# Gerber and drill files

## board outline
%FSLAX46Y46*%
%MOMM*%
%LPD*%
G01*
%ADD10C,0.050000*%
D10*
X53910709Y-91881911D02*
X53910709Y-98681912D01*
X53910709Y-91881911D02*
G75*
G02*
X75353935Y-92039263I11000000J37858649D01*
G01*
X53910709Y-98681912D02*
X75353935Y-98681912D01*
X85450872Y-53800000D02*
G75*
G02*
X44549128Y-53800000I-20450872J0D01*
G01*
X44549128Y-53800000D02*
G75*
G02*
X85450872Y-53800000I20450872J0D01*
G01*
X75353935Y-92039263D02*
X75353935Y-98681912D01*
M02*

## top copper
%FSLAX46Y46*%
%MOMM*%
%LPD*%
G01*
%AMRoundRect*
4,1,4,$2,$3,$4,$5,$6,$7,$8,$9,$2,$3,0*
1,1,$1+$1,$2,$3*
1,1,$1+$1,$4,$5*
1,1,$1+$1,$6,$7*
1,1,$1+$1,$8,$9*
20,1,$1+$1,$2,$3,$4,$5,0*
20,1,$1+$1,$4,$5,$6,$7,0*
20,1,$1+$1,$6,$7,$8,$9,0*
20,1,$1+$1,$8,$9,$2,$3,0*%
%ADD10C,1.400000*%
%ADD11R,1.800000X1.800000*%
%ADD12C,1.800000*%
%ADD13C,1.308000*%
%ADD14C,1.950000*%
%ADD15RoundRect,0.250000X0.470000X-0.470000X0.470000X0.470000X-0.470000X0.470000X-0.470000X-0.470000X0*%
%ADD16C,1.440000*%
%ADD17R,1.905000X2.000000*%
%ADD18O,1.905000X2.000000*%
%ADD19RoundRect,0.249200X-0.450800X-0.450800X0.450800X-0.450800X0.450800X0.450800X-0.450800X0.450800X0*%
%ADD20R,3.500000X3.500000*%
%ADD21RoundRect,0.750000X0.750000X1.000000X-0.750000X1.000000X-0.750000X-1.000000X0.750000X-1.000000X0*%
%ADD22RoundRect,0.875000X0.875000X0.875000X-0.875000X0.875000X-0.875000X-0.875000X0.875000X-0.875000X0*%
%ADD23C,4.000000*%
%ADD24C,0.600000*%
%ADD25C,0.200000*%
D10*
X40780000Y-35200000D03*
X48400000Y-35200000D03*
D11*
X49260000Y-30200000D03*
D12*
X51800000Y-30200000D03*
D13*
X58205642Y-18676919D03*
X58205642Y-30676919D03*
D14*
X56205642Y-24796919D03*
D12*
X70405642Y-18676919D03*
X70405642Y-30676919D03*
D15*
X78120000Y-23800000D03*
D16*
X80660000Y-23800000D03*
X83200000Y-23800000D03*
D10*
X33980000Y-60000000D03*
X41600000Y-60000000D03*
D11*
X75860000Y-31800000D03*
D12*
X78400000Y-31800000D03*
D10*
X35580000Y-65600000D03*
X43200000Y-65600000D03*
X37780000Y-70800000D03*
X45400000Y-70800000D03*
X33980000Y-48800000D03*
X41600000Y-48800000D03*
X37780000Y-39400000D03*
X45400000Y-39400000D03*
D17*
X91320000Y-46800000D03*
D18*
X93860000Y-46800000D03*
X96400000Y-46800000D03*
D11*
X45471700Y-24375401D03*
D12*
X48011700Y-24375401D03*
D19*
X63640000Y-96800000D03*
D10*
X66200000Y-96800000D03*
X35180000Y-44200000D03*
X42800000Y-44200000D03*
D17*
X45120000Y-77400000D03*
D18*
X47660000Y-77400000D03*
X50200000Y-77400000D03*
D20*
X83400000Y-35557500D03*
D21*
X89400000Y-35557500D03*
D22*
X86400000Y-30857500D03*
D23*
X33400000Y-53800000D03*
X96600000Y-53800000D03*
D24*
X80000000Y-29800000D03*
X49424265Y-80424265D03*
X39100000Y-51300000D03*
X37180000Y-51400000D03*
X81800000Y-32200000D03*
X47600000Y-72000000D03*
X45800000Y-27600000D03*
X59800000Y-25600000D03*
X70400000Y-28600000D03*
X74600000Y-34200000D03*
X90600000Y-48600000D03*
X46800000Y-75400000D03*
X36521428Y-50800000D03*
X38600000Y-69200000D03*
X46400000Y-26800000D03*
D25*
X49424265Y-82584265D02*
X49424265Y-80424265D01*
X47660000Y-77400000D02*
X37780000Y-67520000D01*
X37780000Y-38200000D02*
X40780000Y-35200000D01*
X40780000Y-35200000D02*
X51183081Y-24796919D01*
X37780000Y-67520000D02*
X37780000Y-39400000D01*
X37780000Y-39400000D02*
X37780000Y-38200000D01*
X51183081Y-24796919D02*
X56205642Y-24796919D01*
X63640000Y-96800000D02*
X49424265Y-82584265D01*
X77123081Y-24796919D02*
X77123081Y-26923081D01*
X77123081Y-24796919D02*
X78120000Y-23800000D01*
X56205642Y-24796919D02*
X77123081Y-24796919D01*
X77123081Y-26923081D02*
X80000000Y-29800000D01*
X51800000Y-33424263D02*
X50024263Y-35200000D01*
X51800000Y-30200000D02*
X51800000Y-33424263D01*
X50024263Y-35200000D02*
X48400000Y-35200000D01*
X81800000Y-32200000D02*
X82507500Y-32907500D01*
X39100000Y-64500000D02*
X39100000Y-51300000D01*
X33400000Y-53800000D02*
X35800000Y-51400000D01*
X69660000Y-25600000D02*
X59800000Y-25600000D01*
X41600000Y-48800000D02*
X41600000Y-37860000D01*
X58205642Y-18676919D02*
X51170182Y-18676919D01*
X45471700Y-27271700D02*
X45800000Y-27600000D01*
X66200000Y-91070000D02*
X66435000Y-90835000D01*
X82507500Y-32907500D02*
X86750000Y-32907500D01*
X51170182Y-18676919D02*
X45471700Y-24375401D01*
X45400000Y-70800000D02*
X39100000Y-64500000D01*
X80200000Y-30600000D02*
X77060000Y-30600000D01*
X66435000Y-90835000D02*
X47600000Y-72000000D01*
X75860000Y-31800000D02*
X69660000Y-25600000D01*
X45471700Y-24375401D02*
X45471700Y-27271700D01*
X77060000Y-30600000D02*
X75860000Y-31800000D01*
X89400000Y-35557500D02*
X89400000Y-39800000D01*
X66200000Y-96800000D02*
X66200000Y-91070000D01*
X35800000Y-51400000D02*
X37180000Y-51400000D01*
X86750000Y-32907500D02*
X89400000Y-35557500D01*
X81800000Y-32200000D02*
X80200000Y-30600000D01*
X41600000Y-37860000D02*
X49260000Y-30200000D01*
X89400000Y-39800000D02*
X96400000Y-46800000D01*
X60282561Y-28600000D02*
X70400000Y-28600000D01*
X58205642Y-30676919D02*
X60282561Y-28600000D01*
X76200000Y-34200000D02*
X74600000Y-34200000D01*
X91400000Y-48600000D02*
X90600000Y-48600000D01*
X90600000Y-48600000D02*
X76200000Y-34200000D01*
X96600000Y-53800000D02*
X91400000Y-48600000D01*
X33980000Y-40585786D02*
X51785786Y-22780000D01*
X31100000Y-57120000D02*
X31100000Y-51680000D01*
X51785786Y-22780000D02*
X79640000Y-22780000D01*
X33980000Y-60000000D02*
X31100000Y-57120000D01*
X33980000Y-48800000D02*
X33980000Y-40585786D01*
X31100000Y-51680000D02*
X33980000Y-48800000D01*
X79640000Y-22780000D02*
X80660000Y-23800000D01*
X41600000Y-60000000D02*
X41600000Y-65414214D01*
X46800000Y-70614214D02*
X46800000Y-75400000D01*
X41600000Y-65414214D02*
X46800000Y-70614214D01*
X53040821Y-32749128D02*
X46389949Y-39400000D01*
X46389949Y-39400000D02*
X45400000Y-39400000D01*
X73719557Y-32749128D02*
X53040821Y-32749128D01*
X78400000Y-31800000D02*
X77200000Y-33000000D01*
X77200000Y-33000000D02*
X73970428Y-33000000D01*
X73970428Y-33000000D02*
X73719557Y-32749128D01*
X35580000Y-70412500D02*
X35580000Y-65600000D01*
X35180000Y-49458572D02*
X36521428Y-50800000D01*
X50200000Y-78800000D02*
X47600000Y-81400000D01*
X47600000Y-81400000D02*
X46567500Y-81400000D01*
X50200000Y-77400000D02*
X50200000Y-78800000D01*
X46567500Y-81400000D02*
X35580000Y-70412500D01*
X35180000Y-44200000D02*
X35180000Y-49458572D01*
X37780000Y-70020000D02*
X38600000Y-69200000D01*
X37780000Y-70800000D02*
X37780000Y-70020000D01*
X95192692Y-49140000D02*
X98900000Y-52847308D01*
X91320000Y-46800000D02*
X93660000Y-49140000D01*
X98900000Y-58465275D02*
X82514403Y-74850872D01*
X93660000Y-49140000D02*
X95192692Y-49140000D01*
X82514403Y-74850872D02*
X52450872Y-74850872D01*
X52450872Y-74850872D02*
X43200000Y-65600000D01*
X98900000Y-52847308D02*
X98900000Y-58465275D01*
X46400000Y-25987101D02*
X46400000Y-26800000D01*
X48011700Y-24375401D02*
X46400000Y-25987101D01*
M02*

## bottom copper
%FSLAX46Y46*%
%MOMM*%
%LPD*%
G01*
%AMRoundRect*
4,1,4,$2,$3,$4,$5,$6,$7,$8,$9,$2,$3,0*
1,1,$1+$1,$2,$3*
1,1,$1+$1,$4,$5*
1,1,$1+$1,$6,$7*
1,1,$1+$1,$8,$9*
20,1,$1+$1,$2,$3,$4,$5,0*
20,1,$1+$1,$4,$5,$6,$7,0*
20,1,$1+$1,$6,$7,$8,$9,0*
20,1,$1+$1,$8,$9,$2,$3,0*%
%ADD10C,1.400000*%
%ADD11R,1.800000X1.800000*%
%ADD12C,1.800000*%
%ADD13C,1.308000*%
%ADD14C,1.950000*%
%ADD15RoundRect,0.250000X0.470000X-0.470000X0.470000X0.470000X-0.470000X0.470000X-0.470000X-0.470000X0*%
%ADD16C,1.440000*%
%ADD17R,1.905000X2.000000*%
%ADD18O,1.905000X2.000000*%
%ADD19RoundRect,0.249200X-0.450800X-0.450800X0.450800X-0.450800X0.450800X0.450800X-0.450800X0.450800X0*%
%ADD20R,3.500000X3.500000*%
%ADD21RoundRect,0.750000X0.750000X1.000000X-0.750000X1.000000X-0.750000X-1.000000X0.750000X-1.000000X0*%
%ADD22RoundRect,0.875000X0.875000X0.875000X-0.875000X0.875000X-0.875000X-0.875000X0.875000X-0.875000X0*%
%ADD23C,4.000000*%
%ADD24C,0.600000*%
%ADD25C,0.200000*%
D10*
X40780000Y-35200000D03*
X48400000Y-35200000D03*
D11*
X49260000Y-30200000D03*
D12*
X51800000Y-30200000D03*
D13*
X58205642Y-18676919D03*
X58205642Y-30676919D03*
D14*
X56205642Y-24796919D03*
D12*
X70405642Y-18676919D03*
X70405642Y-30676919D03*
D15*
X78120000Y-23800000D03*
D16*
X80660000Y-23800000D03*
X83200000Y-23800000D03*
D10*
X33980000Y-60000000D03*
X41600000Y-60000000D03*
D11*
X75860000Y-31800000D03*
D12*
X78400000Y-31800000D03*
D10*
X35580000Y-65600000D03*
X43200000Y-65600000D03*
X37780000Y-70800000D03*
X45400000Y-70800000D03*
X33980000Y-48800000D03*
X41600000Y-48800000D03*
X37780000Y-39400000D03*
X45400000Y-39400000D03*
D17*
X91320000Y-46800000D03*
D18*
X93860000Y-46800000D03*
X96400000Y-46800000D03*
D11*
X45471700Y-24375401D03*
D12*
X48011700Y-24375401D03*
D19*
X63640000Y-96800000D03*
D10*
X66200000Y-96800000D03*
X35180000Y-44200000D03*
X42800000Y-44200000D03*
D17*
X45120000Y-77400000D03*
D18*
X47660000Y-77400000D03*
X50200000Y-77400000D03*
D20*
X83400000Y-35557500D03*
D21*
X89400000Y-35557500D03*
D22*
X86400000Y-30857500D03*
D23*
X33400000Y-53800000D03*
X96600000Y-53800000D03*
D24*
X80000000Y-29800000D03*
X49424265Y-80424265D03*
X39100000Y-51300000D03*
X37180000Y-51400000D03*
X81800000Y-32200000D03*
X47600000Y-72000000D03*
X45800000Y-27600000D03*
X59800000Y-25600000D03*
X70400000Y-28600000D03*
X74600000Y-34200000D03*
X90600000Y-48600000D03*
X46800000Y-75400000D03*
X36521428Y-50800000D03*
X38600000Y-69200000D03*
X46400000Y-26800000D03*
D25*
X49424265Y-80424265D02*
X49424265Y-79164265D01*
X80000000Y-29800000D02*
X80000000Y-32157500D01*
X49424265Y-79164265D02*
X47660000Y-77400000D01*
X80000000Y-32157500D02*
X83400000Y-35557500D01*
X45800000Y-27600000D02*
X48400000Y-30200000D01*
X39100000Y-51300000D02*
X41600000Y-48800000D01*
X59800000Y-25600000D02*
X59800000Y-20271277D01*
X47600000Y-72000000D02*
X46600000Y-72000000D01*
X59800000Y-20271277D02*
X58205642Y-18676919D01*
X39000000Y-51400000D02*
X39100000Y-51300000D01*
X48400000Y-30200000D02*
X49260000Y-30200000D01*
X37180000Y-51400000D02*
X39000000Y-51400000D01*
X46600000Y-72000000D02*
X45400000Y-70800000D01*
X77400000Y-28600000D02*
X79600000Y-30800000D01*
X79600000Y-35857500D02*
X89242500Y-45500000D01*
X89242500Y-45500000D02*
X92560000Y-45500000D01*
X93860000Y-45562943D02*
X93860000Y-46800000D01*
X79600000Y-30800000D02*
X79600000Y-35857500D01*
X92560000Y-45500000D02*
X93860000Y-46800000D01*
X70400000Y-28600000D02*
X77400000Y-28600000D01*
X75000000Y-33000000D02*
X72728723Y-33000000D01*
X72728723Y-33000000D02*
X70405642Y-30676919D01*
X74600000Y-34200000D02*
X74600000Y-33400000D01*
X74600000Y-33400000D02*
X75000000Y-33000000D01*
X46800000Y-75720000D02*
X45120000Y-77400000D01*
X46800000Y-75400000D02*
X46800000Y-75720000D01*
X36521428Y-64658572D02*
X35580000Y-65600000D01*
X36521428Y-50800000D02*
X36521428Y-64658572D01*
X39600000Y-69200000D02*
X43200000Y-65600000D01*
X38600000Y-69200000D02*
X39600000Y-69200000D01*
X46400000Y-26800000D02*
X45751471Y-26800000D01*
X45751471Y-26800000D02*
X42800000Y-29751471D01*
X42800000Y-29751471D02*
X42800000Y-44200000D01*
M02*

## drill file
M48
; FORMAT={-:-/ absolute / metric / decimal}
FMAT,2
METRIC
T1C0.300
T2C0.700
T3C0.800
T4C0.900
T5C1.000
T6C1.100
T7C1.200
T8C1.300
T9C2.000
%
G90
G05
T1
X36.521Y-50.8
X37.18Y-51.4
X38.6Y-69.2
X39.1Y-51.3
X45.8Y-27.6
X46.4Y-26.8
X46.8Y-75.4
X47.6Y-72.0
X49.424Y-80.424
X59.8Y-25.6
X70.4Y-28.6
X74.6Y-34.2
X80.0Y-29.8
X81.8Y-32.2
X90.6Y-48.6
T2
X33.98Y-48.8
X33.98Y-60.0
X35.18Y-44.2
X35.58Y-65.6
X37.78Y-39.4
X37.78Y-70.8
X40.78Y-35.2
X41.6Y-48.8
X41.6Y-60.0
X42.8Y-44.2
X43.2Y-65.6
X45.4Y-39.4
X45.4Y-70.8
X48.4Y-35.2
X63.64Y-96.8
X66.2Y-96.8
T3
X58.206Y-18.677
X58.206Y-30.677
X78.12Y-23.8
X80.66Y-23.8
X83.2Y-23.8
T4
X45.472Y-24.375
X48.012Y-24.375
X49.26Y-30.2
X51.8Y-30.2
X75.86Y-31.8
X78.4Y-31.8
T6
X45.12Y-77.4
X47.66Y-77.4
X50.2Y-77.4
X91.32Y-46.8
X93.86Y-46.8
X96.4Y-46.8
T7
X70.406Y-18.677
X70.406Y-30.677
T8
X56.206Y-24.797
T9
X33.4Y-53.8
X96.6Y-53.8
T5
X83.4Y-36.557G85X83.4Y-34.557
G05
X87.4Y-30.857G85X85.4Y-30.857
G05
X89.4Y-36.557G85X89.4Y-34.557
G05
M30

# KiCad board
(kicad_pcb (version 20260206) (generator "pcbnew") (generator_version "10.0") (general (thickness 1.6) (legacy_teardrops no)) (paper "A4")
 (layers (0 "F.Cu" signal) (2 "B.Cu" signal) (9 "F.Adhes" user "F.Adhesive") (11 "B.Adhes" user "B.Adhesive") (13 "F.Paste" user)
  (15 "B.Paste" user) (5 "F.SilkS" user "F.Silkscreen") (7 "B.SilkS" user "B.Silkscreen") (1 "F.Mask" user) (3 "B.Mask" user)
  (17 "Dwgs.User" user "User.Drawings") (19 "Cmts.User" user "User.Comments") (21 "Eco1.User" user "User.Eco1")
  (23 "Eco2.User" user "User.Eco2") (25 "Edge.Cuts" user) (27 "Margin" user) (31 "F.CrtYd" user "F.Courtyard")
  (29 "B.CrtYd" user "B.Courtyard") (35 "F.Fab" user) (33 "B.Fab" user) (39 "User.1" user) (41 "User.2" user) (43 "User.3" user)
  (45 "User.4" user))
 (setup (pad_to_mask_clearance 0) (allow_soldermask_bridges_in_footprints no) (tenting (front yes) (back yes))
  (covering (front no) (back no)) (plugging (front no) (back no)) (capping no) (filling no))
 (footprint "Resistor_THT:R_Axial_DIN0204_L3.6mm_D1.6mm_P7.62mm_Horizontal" (layer "F.Cu") (at 40.78 35.2)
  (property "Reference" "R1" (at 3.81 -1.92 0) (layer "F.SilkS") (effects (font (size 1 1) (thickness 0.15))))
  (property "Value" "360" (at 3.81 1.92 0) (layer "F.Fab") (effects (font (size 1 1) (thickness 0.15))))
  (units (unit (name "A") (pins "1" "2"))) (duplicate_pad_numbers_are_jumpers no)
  (pad "1" thru_hole circle (at 0 0) (size 1.4 1.4) (drill 0.7) (layers "*.Cu" "*.Mask") (remove_unused_layers no) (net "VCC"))
  (pad "2" thru_hole circle (at 7.62 0) (size 1.4 1.4) (drill 0.7) (layers "*.Cu" "*.Mask") (remove_unused_layers no) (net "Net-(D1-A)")))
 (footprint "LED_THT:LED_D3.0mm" (layer "F.Cu") (at 49.26 30.2)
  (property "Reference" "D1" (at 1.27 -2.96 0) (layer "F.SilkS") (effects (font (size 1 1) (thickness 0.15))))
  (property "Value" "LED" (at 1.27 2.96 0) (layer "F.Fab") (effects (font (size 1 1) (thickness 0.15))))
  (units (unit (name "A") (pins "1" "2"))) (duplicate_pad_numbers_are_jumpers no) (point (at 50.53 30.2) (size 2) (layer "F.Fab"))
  (pad "1" thru_hole rect (at 0 0) (size 1.8 1.8) (drill 0.9) (layers "*.Cu" "*.Mask") (remove_unused_layers no) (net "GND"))
  (pad "2" thru_hole circle (at 2.54 0) (size 1.8 1.8) (drill 0.9) (layers "*.Cu" "*.Mask") (remove_unused_layers no) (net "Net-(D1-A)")))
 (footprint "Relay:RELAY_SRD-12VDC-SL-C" (layer "F.Cu") (at 64.305642 24.676919)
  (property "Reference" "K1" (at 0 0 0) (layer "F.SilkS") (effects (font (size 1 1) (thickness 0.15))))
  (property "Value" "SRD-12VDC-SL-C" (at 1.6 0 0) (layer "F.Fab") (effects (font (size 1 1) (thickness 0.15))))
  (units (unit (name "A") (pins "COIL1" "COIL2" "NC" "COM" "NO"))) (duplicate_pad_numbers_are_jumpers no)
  (pad "COIL1" thru_hole circle (at -6.1 -6) (size 1.308 1.308) (drill 0.8) (layers "*.Cu" "*.Mask") (remove_unused_layers no) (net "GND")
   (solder_mask_margin 0.102))
  (pad "COIL2" thru_hole circle (at -6.1 6) (size 1.308 1.308) (drill 0.8) (layers "*.Cu" "*.Mask") (remove_unused_layers no)
   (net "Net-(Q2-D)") (solder_mask_margin 0.102))
  (pad "COM" thru_hole circle (at -8.1 0.12) (size 1.95 1.95) (drill 1.3) (layers "*.Cu" "*.Mask") (remove_unused_layers no) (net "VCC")
   (solder_mask_margin 0.102))
  (pad "NC" thru_hole circle (at 6.1 -6) (size 1.8 1.8) (drill 1.2) (layers "*.Cu" "*.Mask") (remove_unused_layers no)
   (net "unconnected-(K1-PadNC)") (solder_mask_margin 0.102))
  (pad "NO" thru_hole circle (at 6.1 6) (size 1.8 1.8) (drill 1.2) (layers "*.Cu" "*.Mask") (remove_unused_layers no) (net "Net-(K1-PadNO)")
   (solder_mask_margin 0.102)))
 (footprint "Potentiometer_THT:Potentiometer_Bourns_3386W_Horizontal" (layer "F.Cu") (at 78.12 23.8)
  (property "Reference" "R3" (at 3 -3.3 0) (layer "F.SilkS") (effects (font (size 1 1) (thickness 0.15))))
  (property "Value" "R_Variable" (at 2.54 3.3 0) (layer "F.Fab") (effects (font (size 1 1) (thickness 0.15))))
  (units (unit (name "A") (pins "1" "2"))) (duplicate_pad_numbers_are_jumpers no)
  (pad "1" thru_hole roundrect (at 0 0 90) (size 1.44 1.44) (drill 0.8) (layers "*.Cu" "*.Mask") (remove_unused_layers no)
   (roundrect_rratio 0.1736111111) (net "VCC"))
  (pad "2" thru_hole circle (at 2.54 0 90) (size 1.44 1.44) (drill 0.8) (layers "*.Cu" "*.Mask") (remove_unused_layers no)
   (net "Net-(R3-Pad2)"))
  (pad "3" thru_hole circle (at 5.08 0 90) (size 1.44 1.44) (drill 0.8) (layers "*.Cu" "*.Mask") (remove_unused_layers no)))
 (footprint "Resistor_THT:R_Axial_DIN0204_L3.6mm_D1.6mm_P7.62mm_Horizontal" (layer "F.Cu") (at 33.98 60)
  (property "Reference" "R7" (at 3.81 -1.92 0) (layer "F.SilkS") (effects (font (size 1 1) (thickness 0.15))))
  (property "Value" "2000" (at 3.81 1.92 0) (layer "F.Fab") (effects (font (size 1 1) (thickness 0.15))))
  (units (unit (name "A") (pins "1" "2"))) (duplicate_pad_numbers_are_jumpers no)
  (pad "1" thru_hole circle (at 0 0) (size 1.4 1.4) (drill 0.7) (layers "*.Cu" "*.Mask") (remove_unused_layers no) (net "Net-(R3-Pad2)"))
  (pad "2" thru_hole circle (at 7.62 0) (size 1.4 1.4) (drill 0.7) (layers "*.Cu" "*.Mask") (remove_unused_layers no) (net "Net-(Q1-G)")))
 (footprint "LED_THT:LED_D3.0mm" (layer "F.Cu") (at 75.86 31.8)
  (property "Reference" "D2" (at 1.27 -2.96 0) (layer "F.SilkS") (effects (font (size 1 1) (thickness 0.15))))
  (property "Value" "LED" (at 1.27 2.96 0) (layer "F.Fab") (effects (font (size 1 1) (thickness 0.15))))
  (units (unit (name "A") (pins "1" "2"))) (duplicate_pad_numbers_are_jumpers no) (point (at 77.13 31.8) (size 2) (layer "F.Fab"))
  (pad "1" thru_hole rect (at 0 0) (size 1.8 1.8) (drill 0.9) (layers "*.Cu" "*.Mask") (remove_unused_layers no) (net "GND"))
  (pad "2" thru_hole circle (at 2.54 0) (size 1.8 1.8) (drill 0.9) (layers "*.Cu" "*.Mask") (remove_unused_layers no) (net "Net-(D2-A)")))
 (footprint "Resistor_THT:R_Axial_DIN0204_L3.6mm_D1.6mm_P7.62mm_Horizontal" (layer "F.Cu") (at 35.58 65.6)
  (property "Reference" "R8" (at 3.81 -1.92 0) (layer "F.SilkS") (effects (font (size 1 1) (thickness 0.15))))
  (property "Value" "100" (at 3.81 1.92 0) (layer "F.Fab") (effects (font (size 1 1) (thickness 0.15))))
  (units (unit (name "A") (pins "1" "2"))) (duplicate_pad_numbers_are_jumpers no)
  (pad "1" thru_hole circle (at 0 0) (size 1.4 1.4) (drill 0.7) (layers "*.Cu" "*.Mask") (remove_unused_layers no) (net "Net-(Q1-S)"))
  (pad "2" thru_hole circle (at 7.62 0) (size 1.4 1.4) (drill 0.7) (layers "*.Cu" "*.Mask") (remove_unused_layers no) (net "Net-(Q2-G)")))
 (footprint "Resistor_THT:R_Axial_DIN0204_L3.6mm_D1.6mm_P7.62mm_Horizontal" (layer "F.Cu") (at 37.78 70.8)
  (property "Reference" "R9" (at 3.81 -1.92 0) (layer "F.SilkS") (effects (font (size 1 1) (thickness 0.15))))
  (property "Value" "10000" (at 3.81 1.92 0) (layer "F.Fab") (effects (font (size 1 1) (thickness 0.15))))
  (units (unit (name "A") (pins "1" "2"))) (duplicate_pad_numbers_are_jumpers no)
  (pad "1" thru_hole circle (at 0 0) (size 1.4 1.4) (drill 0.7) (layers "*.Cu" "*.Mask") (remove_unused_layers no) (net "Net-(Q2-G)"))
  (pad "2" thru_hole circle (at 7.62 0) (size 1.4 1.4) (drill 0.7) (layers "*.Cu" "*.Mask") (remove_unused_layers no) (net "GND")))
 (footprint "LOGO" (layer "F.Cu") (at 91 68.8 90)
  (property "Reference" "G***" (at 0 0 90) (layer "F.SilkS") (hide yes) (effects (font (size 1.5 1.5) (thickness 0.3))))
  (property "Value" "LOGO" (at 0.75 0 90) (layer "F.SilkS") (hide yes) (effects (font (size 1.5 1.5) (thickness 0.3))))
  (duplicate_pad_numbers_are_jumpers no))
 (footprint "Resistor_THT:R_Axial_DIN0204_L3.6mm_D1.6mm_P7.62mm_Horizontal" (layer "F.Cu") (at 33.98 48.8)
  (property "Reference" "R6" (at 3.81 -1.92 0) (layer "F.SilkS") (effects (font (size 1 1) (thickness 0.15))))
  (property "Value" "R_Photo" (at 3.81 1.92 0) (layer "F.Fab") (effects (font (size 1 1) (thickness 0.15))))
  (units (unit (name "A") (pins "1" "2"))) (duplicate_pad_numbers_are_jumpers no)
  (pad "1" thru_hole circle (at 0 0) (size 1.4 1.4) (drill 0.7) (layers "*.Cu" "*.Mask") (remove_unused_layers no) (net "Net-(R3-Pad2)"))
  (pad "2" thru_hole circle (at 7.62 0) (size 1.4 1.4) (drill 0.7) (layers "*.Cu" "*.Mask") (remove_unused_layers no) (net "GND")))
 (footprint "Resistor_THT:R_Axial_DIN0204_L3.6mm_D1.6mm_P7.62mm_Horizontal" (layer "F.Cu") (at 37.78 39.4)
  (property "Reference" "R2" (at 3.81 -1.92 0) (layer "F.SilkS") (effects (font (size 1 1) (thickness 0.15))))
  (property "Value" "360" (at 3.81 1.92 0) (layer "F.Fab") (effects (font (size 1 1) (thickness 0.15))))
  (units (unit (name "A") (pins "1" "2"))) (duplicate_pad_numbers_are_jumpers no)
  (pad "1" thru_hole circle (at 0 0) (size 1.4 1.4) (drill 0.7) (layers "*.Cu" "*.Mask") (remove_unused_layers no) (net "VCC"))
  (pad "2" thru_hole circle (at 7.62 0) (size 1.4 1.4) (drill 0.7) (layers "*.Cu" "*.Mask") (remove_unused_layers no) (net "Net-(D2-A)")))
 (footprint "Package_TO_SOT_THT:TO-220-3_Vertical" (layer "F.Cu") (at 91.32 46.8)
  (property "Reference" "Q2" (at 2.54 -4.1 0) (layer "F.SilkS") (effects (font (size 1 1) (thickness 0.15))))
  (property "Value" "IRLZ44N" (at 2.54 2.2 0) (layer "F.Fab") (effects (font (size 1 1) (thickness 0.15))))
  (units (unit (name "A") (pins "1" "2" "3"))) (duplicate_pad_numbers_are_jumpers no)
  (pad "1" thru_hole rect (at 0 0) (size 1.905 2) (drill 1.1) (layers "*.Cu" "*.Mask") (remove_unused_layers no) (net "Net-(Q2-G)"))
  (pad "2" thru_hole oval (at 2.54 0) (size 1.905 2) (drill 1.1) (layers "*.Cu" "*.Mask") (remove_unused_layers no) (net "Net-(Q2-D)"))
  (pad "3" thru_hole oval (at 5.08 0) (size 1.905 2) (drill 1.1) (layers "*.Cu" "*.Mask") (remove_unused_layers no) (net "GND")))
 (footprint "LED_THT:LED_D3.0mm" (layer "F.Cu") (at 45.4717 24.375401)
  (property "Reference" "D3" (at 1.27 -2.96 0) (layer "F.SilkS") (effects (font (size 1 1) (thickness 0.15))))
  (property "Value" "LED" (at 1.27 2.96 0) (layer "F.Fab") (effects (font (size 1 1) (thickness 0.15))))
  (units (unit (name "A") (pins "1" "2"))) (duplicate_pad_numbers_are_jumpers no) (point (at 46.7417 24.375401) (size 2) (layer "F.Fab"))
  (pad "1" thru_hole rect (at 0 0) (size 1.8 1.8) (drill 0.9) (layers "*.Cu" "*.Mask") (remove_unused_layers no) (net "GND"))
  (pad "2" thru_hole circle (at 2.54 0) (size 1.8 1.8) (drill 0.9) (layers "*.Cu" "*.Mask") (remove_unused_layers no) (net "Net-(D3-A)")))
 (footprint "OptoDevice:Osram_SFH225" (layer "F.Cu") (at 63.64 96.8)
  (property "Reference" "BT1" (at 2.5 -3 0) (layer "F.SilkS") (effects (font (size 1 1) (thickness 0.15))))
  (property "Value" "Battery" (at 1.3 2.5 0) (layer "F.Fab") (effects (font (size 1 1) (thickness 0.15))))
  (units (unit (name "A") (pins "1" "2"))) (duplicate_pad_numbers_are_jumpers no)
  (pad "1" thru_hole roundrect (at 0 0) (size 1.4 1.4) (drill 0.7) (layers "*.Cu" "*.Mask") (remove_unused_layers no)
   (roundrect_rratio 0.178) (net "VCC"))
  (pad "2" thru_hole circle (at 2.56 0) (size 1.4 1.4) (drill 0.7) (layers "*.Cu" "*.Mask") (remove_unused_layers no) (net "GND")))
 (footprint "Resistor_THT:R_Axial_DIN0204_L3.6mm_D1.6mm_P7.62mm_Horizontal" (layer "F.Cu") (at 35.18 44.2)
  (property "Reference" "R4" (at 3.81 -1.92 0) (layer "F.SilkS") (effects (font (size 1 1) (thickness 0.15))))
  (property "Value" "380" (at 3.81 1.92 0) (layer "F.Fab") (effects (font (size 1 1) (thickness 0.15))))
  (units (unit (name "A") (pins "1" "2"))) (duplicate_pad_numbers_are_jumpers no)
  (pad "1" thru_hole circle (at 0 0) (size 1.4 1.4) (drill 0.7) (layers "*.Cu" "*.Mask") (remove_unused_layers no) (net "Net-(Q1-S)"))
  (pad "2" thru_hole circle (at 7.62 0) (size 1.4 1.4) (drill 0.7) (layers "*.Cu" "*.Mask") (remove_unused_layers no) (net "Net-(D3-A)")))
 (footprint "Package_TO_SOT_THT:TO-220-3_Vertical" (layer "F.Cu") (at 45.12 77.4)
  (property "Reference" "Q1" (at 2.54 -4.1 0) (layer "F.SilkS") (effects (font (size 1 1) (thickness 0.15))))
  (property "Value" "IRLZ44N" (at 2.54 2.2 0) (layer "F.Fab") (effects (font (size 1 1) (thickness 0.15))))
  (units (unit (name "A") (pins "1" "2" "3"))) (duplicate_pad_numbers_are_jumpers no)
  (pad "1" thru_hole rect (at 0 0) (size 1.905 2) (drill 1.1) (layers "*.Cu" "*.Mask") (remove_unused_layers no) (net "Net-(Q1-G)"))
  (pad "2" thru_hole oval (at 2.54 0) (size 1.905 2) (drill 1.1) (layers "*.Cu" "*.Mask") (remove_unused_layers no) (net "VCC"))
  (pad "3" thru_hole oval (at 5.08 0) (size 1.905 2) (drill 1.1) (layers "*.Cu" "*.Mask") (remove_unused_layers no) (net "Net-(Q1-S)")))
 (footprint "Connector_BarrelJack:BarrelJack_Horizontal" (layer "F.Cu") (at 83.4 35.5575 180)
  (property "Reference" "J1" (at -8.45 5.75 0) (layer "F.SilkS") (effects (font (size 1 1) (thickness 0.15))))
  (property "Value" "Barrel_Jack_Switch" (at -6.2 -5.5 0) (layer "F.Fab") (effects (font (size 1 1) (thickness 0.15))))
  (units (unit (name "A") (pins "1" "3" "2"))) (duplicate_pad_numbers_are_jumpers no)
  (pad "1" thru_hole rect (at 0 0 180) (size 3.5 3.5) (drill oval 1 3) (layers "*.Cu" "*.Mask") (remove_unused_layers no) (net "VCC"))
  (pad "2" thru_hole roundrect (at -6 0 180) (size 3 3.5) (drill oval 1 3) (layers "*.Cu" "*.Mask") (remove_unused_layers no)
   (roundrect_rratio 0.25) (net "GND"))
  (pad "3" thru_hole roundrect (at -3 4.7 180) (size 3.5 3.5) (drill oval 3 1) (layers "*.Cu" "*.Mask") (remove_unused_layers no)
   (roundrect_rratio 0.25) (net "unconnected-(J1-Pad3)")))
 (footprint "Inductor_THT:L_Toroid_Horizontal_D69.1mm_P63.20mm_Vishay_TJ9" (layer "F.Cu") (at 33.4 53.8)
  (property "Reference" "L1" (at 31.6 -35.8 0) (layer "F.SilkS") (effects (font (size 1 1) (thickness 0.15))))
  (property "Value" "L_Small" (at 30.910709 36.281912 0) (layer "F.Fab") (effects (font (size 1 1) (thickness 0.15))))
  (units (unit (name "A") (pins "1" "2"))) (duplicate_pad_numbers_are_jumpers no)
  (pad "1" thru_hole circle (at 0 0) (size 4 4) (drill 2) (layers "*.Cu" "*.Mask") (remove_unused_layers no) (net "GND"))
  (pad "2" thru_hole circle (at 63.2 0) (size 4 4) (drill 2) (layers "*.Cu" "*.Mask") (remove_unused_layers no) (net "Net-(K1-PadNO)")))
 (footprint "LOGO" (layer "F.Cu") (at 65 86.945401)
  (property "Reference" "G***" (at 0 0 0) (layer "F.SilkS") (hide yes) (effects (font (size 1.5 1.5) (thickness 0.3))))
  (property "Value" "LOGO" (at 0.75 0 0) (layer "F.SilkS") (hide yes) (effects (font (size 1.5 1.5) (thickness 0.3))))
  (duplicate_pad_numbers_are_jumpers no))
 (gr_line (start 53.910709 91.881911) (end 53.910709 98.681912) (stroke (width 0.05) (type default)) (layer "Edge.Cuts"))
 (gr_arc (start 53.910709 91.881911) (mid 65.2 14.6) (end 75.353935 92.039263) (stroke (width 0.05) (type default)) (layer "Edge.Cuts"))
 (gr_line (start 53.910709 98.681912) (end 75.353935 98.681912) (stroke (width 0.05) (type default)) (layer "Edge.Cuts"))
 (gr_circle (center 65 53.8) (end 71.004308 73.34959) (stroke (width 0.05) (type default)) (fill no) (layer "Edge.Cuts"))
 (gr_line (start 75.353935 92.039263) (end 75.353935 98.681912) (stroke (width 0.05) (type default)) (layer "Edge.Cuts"))
 (segment (start 49.424265 82.584265) (end 49.424265 80.424265) (width 0.2) (layer "F.Cu") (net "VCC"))
 (segment (start 47.66 77.4) (end 37.78 67.52) (width 0.2) (layer "F.Cu") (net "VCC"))
 (segment (start 37.78 38.2) (end 40.78 35.2) (width 0.2) (layer "F.Cu") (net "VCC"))
 (segment (start 40.78 35.2) (end 51.183081 24.796919) (width 0.2) (layer "F.Cu") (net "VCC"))
 (segment (start 37.78 67.52) (end 37.78 39.4) (width 0.2) (layer "F.Cu") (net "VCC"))
 (segment (start 37.78 39.4) (end 37.78 38.2) (width 0.2) (layer "F.Cu") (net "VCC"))
 (segment (start 51.183081 24.796919) (end 56.205642 24.796919) (width 0.2) (layer "F.Cu") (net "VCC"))
 (segment (start 63.64 96.8) (end 49.424265 82.584265) (width 0.2) (layer "F.Cu") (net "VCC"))
 (segment (start 77.123081 24.796919) (end 77.123081 26.923081) (width 0.2) (layer "F.Cu") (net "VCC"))
 (segment (start 77.123081 24.796919) (end 78.12 23.8) (width 0.2) (layer "F.Cu") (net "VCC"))
 (segment (start 56.205642 24.796919) (end 77.123081 24.796919) (width 0.2) (layer "F.Cu") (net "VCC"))
 (segment (start 77.123081 26.923081) (end 80 29.8) (width 0.2) (layer "F.Cu") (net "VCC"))
 (via (at 80 29.8) (size 0.6) (drill 0.3) (layers "F.Cu" "B.Cu") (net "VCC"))
 (via (at 49.424265 80.424265) (size 0.6) (drill 0.3) (layers "F.Cu" "B.Cu") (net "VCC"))
 (segment (start 49.424265 80.424265) (end 49.424265 79.164265) (width 0.2) (layer "B.Cu") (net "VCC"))
 (segment (start 80 29.8) (end 80 32.1575) (width 0.2) (layer "B.Cu") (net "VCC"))
 (segment (start 49.424265 79.164265) (end 47.66 77.4) (width 0.2) (layer "B.Cu") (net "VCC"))
 (segment (start 80 32.1575) (end 83.4 35.5575) (width 0.2) (layer "B.Cu") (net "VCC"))
 (segment (start 51.8 33.424263) (end 50.024263 35.2) (width 0.2) (layer "F.Cu") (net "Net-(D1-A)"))
 (segment (start 51.8 30.2) (end 51.8 33.424263) (width 0.2) (layer "F.Cu") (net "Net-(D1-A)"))
 (segment (start 50.024263 35.2) (end 48.4 35.2) (width 0.2) (layer "F.Cu") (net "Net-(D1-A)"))
 (segment (start 81.8 32.2) (end 82.5075 32.9075) (width 0.2) (layer "F.Cu") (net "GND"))
 (segment (start 39.1 64.5) (end 39.1 51.3) (width 0.2) (layer "F.Cu") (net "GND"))
 (segment (start 33.4 53.8) (end 35.8 51.4) (width 0.2) (layer "F.Cu") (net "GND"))
 (segment (start 69.66 25.6) (end 59.8 25.6) (width 0.2) (layer "F.Cu") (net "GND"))
 (segment (start 41.6 48.8) (end 41.6 37.86) (width 0.2) (layer "F.Cu") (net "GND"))
 (segment (start 58.205642 18.676919) (end 51.170182 18.676919) (width 0.2) (layer "F.Cu") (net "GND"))
 (segment (start 45.4717 27.2717) (end 45.8 27.6) (width 0.2) (layer "F.Cu") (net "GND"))
 (segment (start 66.2 91.07) (end 66.435 90.835) (width 0.2) (layer "F.Cu") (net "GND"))
 (segment (start 82.5075 32.9075) (end 86.75 32.9075) (width 0.2) (layer "F.Cu") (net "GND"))
 (segment (start 51.170182 18.676919) (end 45.4717 24.375401) (width 0.2) (layer "F.Cu") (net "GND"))
 (segment (start 45.4 70.8) (end 39.1 64.5) (width 0.2) (layer "F.Cu") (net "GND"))
 (segment (start 80.2 30.6) (end 77.06 30.6) (width 0.2) (layer "F.Cu") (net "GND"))
 (segment (start 66.435 90.835) (end 47.6 72) (width 0.2) (layer "F.Cu") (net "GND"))
 (segment (start 75.86 31.8) (end 69.66 25.6) (width 0.2) (layer "F.Cu") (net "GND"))
 (segment (start 45.4717 24.375401) (end 45.4717 27.2717) (width 0.2) (layer "F.Cu") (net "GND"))
 (segment (start 77.06 30.6) (end 75.86 31.8) (width 0.2) (layer "F.Cu") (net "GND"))
 (segment (start 89.4 35.5575) (end 89.4 39.8) (width 0.2) (layer "F.Cu") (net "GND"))
 (segment (start 66.2 96.8) (end 66.2 91.07) (width 0.2) (layer "F.Cu") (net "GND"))
 (segment (start 35.8 51.4) (end 37.18 51.4) (width 0.2) (layer "F.Cu") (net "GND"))
 (segment (start 86.75 32.9075) (end 89.4 35.5575) (width 0.2) (layer "F.Cu") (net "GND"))
 (segment (start 81.8 32.2) (end 80.2 30.6) (width 0.2) (layer "F.Cu") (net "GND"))
 (segment (start 41.6 37.86) (end 49.26 30.2) (width 0.2) (layer "F.Cu") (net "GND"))
 (segment (start 89.4 39.8) (end 96.4 46.8) (width 0.2) (layer "F.Cu") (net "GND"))
 (via (at 39.1 51.3) (size 0.6) (drill 0.3) (layers "F.Cu" "B.Cu") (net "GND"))
 (via (at 37.18 51.4) (size 0.6) (drill 0.3) (layers "F.Cu" "B.Cu") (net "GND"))
 (via (at 81.8 32.2) (size 0.6) (drill 0.3) (layers "F.Cu" "B.Cu") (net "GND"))
 (via (at 47.6 72) (size 0.6) (drill 0.3) (layers "F.Cu" "B.Cu") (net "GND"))
 (via (at 45.8 27.6) (size 0.6) (drill 0.3) (layers "F.Cu" "B.Cu") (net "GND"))
 (via (at 59.8 25.6) (size 0.6) (drill 0.3) (layers "F.Cu" "B.Cu") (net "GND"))
 (segment (start 45.8 27.6) (end 48.4 30.2) (width 0.2) (layer "B.Cu") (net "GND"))
 (segment (start 39.1 51.3) (end 41.6 48.8) (width 0.2) (layer "B.Cu") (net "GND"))
 (segment (start 59.8 25.6) (end 59.8 20.271277) (width 0.2) (layer "B.Cu") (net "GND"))
 (segment (start 47.6 72) (end 46.6 72) (width 0.2) (layer "B.Cu") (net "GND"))
 (segment (start 59.8 20.271277) (end 58.205642 18.676919) (width 0.2) (layer "B.Cu") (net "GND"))
 (segment (start 39 51.4) (end 39.1 51.3) (width 0.2) (layer "B.Cu") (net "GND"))
 (segment (start 48.4 30.2) (end 49.26 30.2) (width 0.2) (layer "B.Cu") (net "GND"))
 (segment (start 37.18 51.4) (end 39 51.4) (width 0.2) (layer "B.Cu") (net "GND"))
 (segment (start 46.6 72) (end 45.4 70.8) (width 0.2) (layer "B.Cu") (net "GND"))
 (segment (start 60.282561 28.6) (end 70.4 28.6) (width 0.2) (layer "F.Cu") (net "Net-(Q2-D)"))
 (segment (start 58.205642 30.676919) (end 60.282561 28.6) (width 0.2) (layer "F.Cu") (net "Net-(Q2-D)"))
 (via (at 70.4 28.6) (size 0.6) (drill 0.3) (layers "F.Cu" "B.Cu") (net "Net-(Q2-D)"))
 (segment (start 77.4 28.6) (end 79.6 30.8) (width 0.2) (layer "B.Cu") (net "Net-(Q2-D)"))
 (segment (start 79.6 35.8575) (end 89.2425 45.5) (width 0.2) (layer "B.Cu") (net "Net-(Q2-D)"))
 (segment (start 89.2425 45.5) (end 92.56 45.5) (width 0.2) (layer "B.Cu") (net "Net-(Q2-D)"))
 (segment (start 93.86 45.562943) (end 93.86 46.8) (width 0.2) (layer "B.Cu") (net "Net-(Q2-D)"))
 (segment (start 79.6 30.8) (end 79.6 35.8575) (width 0.2) (layer "B.Cu") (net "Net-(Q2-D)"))
 (segment (start 92.56 45.5) (end 93.86 46.8) (width 0.2) (layer "B.Cu") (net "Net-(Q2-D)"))
 (segment (start 70.4 28.6) (end 77.4 28.6) (width 0.2) (layer "B.Cu") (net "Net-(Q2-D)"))
 (segment (start 76.2 34.2) (end 74.6 34.2) (width 0.2) (layer "F.Cu") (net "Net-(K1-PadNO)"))
 (segment (start 91.4 48.6) (end 90.6 48.6) (width 0.2) (layer "F.Cu") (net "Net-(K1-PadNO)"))
 (segment (start 90.6 48.6) (end 76.2 34.2) (width 0.2) (layer "F.Cu") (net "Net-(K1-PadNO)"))
 (segment (start 96.6 53.8) (end 91.4 48.6) (width 0.2) (layer "F.Cu") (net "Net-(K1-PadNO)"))
 (via (at 74.6 34.2) (size 0.6) (drill 0.3) (layers "F.Cu" "B.Cu") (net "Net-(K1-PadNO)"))
 (via (at 90.6 48.6) (size 0.6) (drill 0.3) (layers "F.Cu" "B.Cu") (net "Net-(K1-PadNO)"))
 (segment (start 75 33) (end 72.728723 33) (width 0.2) (layer "B.Cu") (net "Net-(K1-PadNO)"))
 (segment (start 72.728723 33) (end 70.405642 30.676919) (width 0.2) (layer "B.Cu") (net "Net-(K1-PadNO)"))
 (segment (start 74.6 34.2) (end 74.6 33.4) (width 0.2) (layer "B.Cu") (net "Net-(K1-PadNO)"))
 (segment (start 74.6 33.4) (end 75 33) (width 0.2) (layer "B.Cu") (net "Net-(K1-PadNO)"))
 (segment (start 33.98 40.585786) (end 51.785786 22.78) (width 0.2) (layer "F.Cu") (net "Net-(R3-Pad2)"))
 (segment (start 31.1 57.12) (end 31.1 51.68) (width 0.2) (layer "F.Cu") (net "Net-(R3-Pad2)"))
 (segment (start 51.785786 22.78) (end 79.64 22.78) (width 0.2) (layer "F.Cu") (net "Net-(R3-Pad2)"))
 (segment (start 33.98 60) (end 31.1 57.12) (width 0.2) (layer "F.Cu") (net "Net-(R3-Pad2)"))
 (segment (start 33.98 48.8) (end 33.98 40.585786) (width 0.2) (layer "F.Cu") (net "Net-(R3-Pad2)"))
 (segment (start 31.1 51.68) (end 33.98 48.8) (width 0.2) (layer "F.Cu") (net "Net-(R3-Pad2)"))
 (segment (start 79.64 22.78) (end 80.66 23.8) (width 0.2) (layer "F.Cu") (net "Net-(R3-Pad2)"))
 (segment (start 41.6 60) (end 41.6 65.414214) (width 0.2) (layer "F.Cu") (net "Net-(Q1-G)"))
 (segment (start 46.8 70.614214) (end 46.8 75.4) (width 0.2) (layer "F.Cu") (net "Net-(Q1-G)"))
 (segment (start 41.6 65.414214) (end 46.8 70.614214) (width 0.2) (layer "F.Cu") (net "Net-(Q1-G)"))
 (via (at 46.8 75.4) (size 0.6) (drill 0.3) (layers "F.Cu" "B.Cu") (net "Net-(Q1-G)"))
 (segment (start 46.8 75.72) (end 45.12 77.4) (width 0.2) (layer "B.Cu") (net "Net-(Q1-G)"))
 (segment (start 46.8 75.4) (end 46.8 75.72) (width 0.2) (layer "B.Cu") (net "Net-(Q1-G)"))
 (segment (start 53.040821 32.749128) (end 46.389949 39.4) (width 0.2) (layer "F.Cu") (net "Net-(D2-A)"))
 (segment (start 46.389949 39.4) (end 45.4 39.4) (width 0.2) (layer "F.Cu") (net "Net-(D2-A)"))
 (segment (start 73.719557 32.749128) (end 53.040821 32.749128) (width 0.2) (layer "F.Cu") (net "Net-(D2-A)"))
 (segment (start 78.4 31.8) (end 77.2 33) (width 0.2) (layer "F.Cu") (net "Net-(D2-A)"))
 (segment (start 77.2 33) (end 73.970428 33) (width 0.2) (layer "F.Cu") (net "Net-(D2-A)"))
 (segment (start 73.970428 33) (end 73.719557 32.749128) (width 0.2) (layer "F.Cu") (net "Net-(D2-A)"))
 (segment (start 35.58 70.4125) (end 35.58 65.6) (width 0.2) (layer "F.Cu") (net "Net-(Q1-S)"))
 (segment (start 35.18 49.458572) (end 36.521428 50.8) (width 0.2) (layer "F.Cu") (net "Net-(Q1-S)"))
 (segment (start 50.2 78.8) (end 47.6 81.4) (width 0.2) (layer "F.Cu") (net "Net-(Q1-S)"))
 (segment (start 47.6 81.4) (end 46.5675 81.4) (width 0.2) (layer "F.Cu") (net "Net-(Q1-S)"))
 (segment (start 50.2 77.4) (end 50.2 78.8) (width 0.2) (layer "F.Cu") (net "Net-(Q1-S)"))
 (segment (start 46.5675 81.4) (end 35.58 70.4125) (width 0.2) (layer "F.Cu") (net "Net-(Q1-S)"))
 (segment (start 35.18 44.2) (end 35.18 49.458572) (width 0.2) (layer "F.Cu") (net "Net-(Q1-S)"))
 (via (at 36.521428 50.8) (size 0.6) (drill 0.3) (layers "F.Cu" "B.Cu") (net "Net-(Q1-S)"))
 (segment (start 36.521428 64.658572) (end 35.58 65.6) (width 0.2) (layer "B.Cu") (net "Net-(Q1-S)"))
 (segment (start 36.521428 50.8) (end 36.521428 64.658572) (width 0.2) (layer "B.Cu") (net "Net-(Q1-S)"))
 (segment (start 37.78 70.02) (end 38.6 69.2) (width 0.2) (layer "F.Cu") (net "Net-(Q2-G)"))
 (segment (start 37.78 70.8) (end 37.78 70.02) (width 0.2) (layer "F.Cu") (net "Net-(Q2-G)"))
 (segment (start 95.192692 49.14) (end 98.9 52.847308) (width 0.2) (layer "F.Cu") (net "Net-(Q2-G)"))
 (segment (start 91.32 46.8) (end 93.66 49.14) (width 0.2) (layer "F.Cu") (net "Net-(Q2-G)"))
 (segment (start 98.9 58.465275) (end 82.514403 74.850872) (width 0.2) (layer "F.Cu") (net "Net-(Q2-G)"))
 (segment (start 93.66 49.14) (end 95.192692 49.14) (width 0.2) (layer "F.Cu") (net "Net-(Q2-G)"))
 (segment (start 82.514403 74.850872) (end 52.450872 74.850872) (width 0.2) (layer "F.Cu") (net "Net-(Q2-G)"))
 (segment (start 52.450872 74.850872) (end 43.2 65.6) (width 0.2) (layer "F.Cu") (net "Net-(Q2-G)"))
 (segment (start 98.9 52.847308) (end 98.9 58.465275) (width 0.2) (layer "F.Cu") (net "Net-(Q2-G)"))
 (via (at 38.6 69.2) (size 0.6) (drill 0.3) (layers "F.Cu" "B.Cu") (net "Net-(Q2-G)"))
 (segment (start 39.6 69.2) (end 43.2 65.6) (width 0.2) (layer "B.Cu") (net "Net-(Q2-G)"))
 (segment (start 38.6 69.2) (end 39.6 69.2) (width 0.2) (layer "B.Cu") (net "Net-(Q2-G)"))
 (segment (start 46.4 25.987101) (end 46.4 26.8) (width 0.2) (layer "F.Cu") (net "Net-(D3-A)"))
 (segment (start 48.0117 24.375401) (end 46.4 25.987101) (width 0.2) (layer "F.Cu") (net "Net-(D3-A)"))
 (via (at 46.4 26.8) (size 0.6) (drill 0.3) (layers "F.Cu" "B.Cu") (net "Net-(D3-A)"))
 (segment (start 46.4 26.8) (end 45.751471 26.8) (width 0.2) (layer "B.Cu") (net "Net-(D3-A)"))
 (segment (start 45.751471 26.8) (end 42.8 29.751471) (width 0.2) (layer "B.Cu") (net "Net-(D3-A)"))
 (segment (start 42.8 29.751471) (end 42.8 44.2) (width 0.2) (layer "B.Cu") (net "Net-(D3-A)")))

